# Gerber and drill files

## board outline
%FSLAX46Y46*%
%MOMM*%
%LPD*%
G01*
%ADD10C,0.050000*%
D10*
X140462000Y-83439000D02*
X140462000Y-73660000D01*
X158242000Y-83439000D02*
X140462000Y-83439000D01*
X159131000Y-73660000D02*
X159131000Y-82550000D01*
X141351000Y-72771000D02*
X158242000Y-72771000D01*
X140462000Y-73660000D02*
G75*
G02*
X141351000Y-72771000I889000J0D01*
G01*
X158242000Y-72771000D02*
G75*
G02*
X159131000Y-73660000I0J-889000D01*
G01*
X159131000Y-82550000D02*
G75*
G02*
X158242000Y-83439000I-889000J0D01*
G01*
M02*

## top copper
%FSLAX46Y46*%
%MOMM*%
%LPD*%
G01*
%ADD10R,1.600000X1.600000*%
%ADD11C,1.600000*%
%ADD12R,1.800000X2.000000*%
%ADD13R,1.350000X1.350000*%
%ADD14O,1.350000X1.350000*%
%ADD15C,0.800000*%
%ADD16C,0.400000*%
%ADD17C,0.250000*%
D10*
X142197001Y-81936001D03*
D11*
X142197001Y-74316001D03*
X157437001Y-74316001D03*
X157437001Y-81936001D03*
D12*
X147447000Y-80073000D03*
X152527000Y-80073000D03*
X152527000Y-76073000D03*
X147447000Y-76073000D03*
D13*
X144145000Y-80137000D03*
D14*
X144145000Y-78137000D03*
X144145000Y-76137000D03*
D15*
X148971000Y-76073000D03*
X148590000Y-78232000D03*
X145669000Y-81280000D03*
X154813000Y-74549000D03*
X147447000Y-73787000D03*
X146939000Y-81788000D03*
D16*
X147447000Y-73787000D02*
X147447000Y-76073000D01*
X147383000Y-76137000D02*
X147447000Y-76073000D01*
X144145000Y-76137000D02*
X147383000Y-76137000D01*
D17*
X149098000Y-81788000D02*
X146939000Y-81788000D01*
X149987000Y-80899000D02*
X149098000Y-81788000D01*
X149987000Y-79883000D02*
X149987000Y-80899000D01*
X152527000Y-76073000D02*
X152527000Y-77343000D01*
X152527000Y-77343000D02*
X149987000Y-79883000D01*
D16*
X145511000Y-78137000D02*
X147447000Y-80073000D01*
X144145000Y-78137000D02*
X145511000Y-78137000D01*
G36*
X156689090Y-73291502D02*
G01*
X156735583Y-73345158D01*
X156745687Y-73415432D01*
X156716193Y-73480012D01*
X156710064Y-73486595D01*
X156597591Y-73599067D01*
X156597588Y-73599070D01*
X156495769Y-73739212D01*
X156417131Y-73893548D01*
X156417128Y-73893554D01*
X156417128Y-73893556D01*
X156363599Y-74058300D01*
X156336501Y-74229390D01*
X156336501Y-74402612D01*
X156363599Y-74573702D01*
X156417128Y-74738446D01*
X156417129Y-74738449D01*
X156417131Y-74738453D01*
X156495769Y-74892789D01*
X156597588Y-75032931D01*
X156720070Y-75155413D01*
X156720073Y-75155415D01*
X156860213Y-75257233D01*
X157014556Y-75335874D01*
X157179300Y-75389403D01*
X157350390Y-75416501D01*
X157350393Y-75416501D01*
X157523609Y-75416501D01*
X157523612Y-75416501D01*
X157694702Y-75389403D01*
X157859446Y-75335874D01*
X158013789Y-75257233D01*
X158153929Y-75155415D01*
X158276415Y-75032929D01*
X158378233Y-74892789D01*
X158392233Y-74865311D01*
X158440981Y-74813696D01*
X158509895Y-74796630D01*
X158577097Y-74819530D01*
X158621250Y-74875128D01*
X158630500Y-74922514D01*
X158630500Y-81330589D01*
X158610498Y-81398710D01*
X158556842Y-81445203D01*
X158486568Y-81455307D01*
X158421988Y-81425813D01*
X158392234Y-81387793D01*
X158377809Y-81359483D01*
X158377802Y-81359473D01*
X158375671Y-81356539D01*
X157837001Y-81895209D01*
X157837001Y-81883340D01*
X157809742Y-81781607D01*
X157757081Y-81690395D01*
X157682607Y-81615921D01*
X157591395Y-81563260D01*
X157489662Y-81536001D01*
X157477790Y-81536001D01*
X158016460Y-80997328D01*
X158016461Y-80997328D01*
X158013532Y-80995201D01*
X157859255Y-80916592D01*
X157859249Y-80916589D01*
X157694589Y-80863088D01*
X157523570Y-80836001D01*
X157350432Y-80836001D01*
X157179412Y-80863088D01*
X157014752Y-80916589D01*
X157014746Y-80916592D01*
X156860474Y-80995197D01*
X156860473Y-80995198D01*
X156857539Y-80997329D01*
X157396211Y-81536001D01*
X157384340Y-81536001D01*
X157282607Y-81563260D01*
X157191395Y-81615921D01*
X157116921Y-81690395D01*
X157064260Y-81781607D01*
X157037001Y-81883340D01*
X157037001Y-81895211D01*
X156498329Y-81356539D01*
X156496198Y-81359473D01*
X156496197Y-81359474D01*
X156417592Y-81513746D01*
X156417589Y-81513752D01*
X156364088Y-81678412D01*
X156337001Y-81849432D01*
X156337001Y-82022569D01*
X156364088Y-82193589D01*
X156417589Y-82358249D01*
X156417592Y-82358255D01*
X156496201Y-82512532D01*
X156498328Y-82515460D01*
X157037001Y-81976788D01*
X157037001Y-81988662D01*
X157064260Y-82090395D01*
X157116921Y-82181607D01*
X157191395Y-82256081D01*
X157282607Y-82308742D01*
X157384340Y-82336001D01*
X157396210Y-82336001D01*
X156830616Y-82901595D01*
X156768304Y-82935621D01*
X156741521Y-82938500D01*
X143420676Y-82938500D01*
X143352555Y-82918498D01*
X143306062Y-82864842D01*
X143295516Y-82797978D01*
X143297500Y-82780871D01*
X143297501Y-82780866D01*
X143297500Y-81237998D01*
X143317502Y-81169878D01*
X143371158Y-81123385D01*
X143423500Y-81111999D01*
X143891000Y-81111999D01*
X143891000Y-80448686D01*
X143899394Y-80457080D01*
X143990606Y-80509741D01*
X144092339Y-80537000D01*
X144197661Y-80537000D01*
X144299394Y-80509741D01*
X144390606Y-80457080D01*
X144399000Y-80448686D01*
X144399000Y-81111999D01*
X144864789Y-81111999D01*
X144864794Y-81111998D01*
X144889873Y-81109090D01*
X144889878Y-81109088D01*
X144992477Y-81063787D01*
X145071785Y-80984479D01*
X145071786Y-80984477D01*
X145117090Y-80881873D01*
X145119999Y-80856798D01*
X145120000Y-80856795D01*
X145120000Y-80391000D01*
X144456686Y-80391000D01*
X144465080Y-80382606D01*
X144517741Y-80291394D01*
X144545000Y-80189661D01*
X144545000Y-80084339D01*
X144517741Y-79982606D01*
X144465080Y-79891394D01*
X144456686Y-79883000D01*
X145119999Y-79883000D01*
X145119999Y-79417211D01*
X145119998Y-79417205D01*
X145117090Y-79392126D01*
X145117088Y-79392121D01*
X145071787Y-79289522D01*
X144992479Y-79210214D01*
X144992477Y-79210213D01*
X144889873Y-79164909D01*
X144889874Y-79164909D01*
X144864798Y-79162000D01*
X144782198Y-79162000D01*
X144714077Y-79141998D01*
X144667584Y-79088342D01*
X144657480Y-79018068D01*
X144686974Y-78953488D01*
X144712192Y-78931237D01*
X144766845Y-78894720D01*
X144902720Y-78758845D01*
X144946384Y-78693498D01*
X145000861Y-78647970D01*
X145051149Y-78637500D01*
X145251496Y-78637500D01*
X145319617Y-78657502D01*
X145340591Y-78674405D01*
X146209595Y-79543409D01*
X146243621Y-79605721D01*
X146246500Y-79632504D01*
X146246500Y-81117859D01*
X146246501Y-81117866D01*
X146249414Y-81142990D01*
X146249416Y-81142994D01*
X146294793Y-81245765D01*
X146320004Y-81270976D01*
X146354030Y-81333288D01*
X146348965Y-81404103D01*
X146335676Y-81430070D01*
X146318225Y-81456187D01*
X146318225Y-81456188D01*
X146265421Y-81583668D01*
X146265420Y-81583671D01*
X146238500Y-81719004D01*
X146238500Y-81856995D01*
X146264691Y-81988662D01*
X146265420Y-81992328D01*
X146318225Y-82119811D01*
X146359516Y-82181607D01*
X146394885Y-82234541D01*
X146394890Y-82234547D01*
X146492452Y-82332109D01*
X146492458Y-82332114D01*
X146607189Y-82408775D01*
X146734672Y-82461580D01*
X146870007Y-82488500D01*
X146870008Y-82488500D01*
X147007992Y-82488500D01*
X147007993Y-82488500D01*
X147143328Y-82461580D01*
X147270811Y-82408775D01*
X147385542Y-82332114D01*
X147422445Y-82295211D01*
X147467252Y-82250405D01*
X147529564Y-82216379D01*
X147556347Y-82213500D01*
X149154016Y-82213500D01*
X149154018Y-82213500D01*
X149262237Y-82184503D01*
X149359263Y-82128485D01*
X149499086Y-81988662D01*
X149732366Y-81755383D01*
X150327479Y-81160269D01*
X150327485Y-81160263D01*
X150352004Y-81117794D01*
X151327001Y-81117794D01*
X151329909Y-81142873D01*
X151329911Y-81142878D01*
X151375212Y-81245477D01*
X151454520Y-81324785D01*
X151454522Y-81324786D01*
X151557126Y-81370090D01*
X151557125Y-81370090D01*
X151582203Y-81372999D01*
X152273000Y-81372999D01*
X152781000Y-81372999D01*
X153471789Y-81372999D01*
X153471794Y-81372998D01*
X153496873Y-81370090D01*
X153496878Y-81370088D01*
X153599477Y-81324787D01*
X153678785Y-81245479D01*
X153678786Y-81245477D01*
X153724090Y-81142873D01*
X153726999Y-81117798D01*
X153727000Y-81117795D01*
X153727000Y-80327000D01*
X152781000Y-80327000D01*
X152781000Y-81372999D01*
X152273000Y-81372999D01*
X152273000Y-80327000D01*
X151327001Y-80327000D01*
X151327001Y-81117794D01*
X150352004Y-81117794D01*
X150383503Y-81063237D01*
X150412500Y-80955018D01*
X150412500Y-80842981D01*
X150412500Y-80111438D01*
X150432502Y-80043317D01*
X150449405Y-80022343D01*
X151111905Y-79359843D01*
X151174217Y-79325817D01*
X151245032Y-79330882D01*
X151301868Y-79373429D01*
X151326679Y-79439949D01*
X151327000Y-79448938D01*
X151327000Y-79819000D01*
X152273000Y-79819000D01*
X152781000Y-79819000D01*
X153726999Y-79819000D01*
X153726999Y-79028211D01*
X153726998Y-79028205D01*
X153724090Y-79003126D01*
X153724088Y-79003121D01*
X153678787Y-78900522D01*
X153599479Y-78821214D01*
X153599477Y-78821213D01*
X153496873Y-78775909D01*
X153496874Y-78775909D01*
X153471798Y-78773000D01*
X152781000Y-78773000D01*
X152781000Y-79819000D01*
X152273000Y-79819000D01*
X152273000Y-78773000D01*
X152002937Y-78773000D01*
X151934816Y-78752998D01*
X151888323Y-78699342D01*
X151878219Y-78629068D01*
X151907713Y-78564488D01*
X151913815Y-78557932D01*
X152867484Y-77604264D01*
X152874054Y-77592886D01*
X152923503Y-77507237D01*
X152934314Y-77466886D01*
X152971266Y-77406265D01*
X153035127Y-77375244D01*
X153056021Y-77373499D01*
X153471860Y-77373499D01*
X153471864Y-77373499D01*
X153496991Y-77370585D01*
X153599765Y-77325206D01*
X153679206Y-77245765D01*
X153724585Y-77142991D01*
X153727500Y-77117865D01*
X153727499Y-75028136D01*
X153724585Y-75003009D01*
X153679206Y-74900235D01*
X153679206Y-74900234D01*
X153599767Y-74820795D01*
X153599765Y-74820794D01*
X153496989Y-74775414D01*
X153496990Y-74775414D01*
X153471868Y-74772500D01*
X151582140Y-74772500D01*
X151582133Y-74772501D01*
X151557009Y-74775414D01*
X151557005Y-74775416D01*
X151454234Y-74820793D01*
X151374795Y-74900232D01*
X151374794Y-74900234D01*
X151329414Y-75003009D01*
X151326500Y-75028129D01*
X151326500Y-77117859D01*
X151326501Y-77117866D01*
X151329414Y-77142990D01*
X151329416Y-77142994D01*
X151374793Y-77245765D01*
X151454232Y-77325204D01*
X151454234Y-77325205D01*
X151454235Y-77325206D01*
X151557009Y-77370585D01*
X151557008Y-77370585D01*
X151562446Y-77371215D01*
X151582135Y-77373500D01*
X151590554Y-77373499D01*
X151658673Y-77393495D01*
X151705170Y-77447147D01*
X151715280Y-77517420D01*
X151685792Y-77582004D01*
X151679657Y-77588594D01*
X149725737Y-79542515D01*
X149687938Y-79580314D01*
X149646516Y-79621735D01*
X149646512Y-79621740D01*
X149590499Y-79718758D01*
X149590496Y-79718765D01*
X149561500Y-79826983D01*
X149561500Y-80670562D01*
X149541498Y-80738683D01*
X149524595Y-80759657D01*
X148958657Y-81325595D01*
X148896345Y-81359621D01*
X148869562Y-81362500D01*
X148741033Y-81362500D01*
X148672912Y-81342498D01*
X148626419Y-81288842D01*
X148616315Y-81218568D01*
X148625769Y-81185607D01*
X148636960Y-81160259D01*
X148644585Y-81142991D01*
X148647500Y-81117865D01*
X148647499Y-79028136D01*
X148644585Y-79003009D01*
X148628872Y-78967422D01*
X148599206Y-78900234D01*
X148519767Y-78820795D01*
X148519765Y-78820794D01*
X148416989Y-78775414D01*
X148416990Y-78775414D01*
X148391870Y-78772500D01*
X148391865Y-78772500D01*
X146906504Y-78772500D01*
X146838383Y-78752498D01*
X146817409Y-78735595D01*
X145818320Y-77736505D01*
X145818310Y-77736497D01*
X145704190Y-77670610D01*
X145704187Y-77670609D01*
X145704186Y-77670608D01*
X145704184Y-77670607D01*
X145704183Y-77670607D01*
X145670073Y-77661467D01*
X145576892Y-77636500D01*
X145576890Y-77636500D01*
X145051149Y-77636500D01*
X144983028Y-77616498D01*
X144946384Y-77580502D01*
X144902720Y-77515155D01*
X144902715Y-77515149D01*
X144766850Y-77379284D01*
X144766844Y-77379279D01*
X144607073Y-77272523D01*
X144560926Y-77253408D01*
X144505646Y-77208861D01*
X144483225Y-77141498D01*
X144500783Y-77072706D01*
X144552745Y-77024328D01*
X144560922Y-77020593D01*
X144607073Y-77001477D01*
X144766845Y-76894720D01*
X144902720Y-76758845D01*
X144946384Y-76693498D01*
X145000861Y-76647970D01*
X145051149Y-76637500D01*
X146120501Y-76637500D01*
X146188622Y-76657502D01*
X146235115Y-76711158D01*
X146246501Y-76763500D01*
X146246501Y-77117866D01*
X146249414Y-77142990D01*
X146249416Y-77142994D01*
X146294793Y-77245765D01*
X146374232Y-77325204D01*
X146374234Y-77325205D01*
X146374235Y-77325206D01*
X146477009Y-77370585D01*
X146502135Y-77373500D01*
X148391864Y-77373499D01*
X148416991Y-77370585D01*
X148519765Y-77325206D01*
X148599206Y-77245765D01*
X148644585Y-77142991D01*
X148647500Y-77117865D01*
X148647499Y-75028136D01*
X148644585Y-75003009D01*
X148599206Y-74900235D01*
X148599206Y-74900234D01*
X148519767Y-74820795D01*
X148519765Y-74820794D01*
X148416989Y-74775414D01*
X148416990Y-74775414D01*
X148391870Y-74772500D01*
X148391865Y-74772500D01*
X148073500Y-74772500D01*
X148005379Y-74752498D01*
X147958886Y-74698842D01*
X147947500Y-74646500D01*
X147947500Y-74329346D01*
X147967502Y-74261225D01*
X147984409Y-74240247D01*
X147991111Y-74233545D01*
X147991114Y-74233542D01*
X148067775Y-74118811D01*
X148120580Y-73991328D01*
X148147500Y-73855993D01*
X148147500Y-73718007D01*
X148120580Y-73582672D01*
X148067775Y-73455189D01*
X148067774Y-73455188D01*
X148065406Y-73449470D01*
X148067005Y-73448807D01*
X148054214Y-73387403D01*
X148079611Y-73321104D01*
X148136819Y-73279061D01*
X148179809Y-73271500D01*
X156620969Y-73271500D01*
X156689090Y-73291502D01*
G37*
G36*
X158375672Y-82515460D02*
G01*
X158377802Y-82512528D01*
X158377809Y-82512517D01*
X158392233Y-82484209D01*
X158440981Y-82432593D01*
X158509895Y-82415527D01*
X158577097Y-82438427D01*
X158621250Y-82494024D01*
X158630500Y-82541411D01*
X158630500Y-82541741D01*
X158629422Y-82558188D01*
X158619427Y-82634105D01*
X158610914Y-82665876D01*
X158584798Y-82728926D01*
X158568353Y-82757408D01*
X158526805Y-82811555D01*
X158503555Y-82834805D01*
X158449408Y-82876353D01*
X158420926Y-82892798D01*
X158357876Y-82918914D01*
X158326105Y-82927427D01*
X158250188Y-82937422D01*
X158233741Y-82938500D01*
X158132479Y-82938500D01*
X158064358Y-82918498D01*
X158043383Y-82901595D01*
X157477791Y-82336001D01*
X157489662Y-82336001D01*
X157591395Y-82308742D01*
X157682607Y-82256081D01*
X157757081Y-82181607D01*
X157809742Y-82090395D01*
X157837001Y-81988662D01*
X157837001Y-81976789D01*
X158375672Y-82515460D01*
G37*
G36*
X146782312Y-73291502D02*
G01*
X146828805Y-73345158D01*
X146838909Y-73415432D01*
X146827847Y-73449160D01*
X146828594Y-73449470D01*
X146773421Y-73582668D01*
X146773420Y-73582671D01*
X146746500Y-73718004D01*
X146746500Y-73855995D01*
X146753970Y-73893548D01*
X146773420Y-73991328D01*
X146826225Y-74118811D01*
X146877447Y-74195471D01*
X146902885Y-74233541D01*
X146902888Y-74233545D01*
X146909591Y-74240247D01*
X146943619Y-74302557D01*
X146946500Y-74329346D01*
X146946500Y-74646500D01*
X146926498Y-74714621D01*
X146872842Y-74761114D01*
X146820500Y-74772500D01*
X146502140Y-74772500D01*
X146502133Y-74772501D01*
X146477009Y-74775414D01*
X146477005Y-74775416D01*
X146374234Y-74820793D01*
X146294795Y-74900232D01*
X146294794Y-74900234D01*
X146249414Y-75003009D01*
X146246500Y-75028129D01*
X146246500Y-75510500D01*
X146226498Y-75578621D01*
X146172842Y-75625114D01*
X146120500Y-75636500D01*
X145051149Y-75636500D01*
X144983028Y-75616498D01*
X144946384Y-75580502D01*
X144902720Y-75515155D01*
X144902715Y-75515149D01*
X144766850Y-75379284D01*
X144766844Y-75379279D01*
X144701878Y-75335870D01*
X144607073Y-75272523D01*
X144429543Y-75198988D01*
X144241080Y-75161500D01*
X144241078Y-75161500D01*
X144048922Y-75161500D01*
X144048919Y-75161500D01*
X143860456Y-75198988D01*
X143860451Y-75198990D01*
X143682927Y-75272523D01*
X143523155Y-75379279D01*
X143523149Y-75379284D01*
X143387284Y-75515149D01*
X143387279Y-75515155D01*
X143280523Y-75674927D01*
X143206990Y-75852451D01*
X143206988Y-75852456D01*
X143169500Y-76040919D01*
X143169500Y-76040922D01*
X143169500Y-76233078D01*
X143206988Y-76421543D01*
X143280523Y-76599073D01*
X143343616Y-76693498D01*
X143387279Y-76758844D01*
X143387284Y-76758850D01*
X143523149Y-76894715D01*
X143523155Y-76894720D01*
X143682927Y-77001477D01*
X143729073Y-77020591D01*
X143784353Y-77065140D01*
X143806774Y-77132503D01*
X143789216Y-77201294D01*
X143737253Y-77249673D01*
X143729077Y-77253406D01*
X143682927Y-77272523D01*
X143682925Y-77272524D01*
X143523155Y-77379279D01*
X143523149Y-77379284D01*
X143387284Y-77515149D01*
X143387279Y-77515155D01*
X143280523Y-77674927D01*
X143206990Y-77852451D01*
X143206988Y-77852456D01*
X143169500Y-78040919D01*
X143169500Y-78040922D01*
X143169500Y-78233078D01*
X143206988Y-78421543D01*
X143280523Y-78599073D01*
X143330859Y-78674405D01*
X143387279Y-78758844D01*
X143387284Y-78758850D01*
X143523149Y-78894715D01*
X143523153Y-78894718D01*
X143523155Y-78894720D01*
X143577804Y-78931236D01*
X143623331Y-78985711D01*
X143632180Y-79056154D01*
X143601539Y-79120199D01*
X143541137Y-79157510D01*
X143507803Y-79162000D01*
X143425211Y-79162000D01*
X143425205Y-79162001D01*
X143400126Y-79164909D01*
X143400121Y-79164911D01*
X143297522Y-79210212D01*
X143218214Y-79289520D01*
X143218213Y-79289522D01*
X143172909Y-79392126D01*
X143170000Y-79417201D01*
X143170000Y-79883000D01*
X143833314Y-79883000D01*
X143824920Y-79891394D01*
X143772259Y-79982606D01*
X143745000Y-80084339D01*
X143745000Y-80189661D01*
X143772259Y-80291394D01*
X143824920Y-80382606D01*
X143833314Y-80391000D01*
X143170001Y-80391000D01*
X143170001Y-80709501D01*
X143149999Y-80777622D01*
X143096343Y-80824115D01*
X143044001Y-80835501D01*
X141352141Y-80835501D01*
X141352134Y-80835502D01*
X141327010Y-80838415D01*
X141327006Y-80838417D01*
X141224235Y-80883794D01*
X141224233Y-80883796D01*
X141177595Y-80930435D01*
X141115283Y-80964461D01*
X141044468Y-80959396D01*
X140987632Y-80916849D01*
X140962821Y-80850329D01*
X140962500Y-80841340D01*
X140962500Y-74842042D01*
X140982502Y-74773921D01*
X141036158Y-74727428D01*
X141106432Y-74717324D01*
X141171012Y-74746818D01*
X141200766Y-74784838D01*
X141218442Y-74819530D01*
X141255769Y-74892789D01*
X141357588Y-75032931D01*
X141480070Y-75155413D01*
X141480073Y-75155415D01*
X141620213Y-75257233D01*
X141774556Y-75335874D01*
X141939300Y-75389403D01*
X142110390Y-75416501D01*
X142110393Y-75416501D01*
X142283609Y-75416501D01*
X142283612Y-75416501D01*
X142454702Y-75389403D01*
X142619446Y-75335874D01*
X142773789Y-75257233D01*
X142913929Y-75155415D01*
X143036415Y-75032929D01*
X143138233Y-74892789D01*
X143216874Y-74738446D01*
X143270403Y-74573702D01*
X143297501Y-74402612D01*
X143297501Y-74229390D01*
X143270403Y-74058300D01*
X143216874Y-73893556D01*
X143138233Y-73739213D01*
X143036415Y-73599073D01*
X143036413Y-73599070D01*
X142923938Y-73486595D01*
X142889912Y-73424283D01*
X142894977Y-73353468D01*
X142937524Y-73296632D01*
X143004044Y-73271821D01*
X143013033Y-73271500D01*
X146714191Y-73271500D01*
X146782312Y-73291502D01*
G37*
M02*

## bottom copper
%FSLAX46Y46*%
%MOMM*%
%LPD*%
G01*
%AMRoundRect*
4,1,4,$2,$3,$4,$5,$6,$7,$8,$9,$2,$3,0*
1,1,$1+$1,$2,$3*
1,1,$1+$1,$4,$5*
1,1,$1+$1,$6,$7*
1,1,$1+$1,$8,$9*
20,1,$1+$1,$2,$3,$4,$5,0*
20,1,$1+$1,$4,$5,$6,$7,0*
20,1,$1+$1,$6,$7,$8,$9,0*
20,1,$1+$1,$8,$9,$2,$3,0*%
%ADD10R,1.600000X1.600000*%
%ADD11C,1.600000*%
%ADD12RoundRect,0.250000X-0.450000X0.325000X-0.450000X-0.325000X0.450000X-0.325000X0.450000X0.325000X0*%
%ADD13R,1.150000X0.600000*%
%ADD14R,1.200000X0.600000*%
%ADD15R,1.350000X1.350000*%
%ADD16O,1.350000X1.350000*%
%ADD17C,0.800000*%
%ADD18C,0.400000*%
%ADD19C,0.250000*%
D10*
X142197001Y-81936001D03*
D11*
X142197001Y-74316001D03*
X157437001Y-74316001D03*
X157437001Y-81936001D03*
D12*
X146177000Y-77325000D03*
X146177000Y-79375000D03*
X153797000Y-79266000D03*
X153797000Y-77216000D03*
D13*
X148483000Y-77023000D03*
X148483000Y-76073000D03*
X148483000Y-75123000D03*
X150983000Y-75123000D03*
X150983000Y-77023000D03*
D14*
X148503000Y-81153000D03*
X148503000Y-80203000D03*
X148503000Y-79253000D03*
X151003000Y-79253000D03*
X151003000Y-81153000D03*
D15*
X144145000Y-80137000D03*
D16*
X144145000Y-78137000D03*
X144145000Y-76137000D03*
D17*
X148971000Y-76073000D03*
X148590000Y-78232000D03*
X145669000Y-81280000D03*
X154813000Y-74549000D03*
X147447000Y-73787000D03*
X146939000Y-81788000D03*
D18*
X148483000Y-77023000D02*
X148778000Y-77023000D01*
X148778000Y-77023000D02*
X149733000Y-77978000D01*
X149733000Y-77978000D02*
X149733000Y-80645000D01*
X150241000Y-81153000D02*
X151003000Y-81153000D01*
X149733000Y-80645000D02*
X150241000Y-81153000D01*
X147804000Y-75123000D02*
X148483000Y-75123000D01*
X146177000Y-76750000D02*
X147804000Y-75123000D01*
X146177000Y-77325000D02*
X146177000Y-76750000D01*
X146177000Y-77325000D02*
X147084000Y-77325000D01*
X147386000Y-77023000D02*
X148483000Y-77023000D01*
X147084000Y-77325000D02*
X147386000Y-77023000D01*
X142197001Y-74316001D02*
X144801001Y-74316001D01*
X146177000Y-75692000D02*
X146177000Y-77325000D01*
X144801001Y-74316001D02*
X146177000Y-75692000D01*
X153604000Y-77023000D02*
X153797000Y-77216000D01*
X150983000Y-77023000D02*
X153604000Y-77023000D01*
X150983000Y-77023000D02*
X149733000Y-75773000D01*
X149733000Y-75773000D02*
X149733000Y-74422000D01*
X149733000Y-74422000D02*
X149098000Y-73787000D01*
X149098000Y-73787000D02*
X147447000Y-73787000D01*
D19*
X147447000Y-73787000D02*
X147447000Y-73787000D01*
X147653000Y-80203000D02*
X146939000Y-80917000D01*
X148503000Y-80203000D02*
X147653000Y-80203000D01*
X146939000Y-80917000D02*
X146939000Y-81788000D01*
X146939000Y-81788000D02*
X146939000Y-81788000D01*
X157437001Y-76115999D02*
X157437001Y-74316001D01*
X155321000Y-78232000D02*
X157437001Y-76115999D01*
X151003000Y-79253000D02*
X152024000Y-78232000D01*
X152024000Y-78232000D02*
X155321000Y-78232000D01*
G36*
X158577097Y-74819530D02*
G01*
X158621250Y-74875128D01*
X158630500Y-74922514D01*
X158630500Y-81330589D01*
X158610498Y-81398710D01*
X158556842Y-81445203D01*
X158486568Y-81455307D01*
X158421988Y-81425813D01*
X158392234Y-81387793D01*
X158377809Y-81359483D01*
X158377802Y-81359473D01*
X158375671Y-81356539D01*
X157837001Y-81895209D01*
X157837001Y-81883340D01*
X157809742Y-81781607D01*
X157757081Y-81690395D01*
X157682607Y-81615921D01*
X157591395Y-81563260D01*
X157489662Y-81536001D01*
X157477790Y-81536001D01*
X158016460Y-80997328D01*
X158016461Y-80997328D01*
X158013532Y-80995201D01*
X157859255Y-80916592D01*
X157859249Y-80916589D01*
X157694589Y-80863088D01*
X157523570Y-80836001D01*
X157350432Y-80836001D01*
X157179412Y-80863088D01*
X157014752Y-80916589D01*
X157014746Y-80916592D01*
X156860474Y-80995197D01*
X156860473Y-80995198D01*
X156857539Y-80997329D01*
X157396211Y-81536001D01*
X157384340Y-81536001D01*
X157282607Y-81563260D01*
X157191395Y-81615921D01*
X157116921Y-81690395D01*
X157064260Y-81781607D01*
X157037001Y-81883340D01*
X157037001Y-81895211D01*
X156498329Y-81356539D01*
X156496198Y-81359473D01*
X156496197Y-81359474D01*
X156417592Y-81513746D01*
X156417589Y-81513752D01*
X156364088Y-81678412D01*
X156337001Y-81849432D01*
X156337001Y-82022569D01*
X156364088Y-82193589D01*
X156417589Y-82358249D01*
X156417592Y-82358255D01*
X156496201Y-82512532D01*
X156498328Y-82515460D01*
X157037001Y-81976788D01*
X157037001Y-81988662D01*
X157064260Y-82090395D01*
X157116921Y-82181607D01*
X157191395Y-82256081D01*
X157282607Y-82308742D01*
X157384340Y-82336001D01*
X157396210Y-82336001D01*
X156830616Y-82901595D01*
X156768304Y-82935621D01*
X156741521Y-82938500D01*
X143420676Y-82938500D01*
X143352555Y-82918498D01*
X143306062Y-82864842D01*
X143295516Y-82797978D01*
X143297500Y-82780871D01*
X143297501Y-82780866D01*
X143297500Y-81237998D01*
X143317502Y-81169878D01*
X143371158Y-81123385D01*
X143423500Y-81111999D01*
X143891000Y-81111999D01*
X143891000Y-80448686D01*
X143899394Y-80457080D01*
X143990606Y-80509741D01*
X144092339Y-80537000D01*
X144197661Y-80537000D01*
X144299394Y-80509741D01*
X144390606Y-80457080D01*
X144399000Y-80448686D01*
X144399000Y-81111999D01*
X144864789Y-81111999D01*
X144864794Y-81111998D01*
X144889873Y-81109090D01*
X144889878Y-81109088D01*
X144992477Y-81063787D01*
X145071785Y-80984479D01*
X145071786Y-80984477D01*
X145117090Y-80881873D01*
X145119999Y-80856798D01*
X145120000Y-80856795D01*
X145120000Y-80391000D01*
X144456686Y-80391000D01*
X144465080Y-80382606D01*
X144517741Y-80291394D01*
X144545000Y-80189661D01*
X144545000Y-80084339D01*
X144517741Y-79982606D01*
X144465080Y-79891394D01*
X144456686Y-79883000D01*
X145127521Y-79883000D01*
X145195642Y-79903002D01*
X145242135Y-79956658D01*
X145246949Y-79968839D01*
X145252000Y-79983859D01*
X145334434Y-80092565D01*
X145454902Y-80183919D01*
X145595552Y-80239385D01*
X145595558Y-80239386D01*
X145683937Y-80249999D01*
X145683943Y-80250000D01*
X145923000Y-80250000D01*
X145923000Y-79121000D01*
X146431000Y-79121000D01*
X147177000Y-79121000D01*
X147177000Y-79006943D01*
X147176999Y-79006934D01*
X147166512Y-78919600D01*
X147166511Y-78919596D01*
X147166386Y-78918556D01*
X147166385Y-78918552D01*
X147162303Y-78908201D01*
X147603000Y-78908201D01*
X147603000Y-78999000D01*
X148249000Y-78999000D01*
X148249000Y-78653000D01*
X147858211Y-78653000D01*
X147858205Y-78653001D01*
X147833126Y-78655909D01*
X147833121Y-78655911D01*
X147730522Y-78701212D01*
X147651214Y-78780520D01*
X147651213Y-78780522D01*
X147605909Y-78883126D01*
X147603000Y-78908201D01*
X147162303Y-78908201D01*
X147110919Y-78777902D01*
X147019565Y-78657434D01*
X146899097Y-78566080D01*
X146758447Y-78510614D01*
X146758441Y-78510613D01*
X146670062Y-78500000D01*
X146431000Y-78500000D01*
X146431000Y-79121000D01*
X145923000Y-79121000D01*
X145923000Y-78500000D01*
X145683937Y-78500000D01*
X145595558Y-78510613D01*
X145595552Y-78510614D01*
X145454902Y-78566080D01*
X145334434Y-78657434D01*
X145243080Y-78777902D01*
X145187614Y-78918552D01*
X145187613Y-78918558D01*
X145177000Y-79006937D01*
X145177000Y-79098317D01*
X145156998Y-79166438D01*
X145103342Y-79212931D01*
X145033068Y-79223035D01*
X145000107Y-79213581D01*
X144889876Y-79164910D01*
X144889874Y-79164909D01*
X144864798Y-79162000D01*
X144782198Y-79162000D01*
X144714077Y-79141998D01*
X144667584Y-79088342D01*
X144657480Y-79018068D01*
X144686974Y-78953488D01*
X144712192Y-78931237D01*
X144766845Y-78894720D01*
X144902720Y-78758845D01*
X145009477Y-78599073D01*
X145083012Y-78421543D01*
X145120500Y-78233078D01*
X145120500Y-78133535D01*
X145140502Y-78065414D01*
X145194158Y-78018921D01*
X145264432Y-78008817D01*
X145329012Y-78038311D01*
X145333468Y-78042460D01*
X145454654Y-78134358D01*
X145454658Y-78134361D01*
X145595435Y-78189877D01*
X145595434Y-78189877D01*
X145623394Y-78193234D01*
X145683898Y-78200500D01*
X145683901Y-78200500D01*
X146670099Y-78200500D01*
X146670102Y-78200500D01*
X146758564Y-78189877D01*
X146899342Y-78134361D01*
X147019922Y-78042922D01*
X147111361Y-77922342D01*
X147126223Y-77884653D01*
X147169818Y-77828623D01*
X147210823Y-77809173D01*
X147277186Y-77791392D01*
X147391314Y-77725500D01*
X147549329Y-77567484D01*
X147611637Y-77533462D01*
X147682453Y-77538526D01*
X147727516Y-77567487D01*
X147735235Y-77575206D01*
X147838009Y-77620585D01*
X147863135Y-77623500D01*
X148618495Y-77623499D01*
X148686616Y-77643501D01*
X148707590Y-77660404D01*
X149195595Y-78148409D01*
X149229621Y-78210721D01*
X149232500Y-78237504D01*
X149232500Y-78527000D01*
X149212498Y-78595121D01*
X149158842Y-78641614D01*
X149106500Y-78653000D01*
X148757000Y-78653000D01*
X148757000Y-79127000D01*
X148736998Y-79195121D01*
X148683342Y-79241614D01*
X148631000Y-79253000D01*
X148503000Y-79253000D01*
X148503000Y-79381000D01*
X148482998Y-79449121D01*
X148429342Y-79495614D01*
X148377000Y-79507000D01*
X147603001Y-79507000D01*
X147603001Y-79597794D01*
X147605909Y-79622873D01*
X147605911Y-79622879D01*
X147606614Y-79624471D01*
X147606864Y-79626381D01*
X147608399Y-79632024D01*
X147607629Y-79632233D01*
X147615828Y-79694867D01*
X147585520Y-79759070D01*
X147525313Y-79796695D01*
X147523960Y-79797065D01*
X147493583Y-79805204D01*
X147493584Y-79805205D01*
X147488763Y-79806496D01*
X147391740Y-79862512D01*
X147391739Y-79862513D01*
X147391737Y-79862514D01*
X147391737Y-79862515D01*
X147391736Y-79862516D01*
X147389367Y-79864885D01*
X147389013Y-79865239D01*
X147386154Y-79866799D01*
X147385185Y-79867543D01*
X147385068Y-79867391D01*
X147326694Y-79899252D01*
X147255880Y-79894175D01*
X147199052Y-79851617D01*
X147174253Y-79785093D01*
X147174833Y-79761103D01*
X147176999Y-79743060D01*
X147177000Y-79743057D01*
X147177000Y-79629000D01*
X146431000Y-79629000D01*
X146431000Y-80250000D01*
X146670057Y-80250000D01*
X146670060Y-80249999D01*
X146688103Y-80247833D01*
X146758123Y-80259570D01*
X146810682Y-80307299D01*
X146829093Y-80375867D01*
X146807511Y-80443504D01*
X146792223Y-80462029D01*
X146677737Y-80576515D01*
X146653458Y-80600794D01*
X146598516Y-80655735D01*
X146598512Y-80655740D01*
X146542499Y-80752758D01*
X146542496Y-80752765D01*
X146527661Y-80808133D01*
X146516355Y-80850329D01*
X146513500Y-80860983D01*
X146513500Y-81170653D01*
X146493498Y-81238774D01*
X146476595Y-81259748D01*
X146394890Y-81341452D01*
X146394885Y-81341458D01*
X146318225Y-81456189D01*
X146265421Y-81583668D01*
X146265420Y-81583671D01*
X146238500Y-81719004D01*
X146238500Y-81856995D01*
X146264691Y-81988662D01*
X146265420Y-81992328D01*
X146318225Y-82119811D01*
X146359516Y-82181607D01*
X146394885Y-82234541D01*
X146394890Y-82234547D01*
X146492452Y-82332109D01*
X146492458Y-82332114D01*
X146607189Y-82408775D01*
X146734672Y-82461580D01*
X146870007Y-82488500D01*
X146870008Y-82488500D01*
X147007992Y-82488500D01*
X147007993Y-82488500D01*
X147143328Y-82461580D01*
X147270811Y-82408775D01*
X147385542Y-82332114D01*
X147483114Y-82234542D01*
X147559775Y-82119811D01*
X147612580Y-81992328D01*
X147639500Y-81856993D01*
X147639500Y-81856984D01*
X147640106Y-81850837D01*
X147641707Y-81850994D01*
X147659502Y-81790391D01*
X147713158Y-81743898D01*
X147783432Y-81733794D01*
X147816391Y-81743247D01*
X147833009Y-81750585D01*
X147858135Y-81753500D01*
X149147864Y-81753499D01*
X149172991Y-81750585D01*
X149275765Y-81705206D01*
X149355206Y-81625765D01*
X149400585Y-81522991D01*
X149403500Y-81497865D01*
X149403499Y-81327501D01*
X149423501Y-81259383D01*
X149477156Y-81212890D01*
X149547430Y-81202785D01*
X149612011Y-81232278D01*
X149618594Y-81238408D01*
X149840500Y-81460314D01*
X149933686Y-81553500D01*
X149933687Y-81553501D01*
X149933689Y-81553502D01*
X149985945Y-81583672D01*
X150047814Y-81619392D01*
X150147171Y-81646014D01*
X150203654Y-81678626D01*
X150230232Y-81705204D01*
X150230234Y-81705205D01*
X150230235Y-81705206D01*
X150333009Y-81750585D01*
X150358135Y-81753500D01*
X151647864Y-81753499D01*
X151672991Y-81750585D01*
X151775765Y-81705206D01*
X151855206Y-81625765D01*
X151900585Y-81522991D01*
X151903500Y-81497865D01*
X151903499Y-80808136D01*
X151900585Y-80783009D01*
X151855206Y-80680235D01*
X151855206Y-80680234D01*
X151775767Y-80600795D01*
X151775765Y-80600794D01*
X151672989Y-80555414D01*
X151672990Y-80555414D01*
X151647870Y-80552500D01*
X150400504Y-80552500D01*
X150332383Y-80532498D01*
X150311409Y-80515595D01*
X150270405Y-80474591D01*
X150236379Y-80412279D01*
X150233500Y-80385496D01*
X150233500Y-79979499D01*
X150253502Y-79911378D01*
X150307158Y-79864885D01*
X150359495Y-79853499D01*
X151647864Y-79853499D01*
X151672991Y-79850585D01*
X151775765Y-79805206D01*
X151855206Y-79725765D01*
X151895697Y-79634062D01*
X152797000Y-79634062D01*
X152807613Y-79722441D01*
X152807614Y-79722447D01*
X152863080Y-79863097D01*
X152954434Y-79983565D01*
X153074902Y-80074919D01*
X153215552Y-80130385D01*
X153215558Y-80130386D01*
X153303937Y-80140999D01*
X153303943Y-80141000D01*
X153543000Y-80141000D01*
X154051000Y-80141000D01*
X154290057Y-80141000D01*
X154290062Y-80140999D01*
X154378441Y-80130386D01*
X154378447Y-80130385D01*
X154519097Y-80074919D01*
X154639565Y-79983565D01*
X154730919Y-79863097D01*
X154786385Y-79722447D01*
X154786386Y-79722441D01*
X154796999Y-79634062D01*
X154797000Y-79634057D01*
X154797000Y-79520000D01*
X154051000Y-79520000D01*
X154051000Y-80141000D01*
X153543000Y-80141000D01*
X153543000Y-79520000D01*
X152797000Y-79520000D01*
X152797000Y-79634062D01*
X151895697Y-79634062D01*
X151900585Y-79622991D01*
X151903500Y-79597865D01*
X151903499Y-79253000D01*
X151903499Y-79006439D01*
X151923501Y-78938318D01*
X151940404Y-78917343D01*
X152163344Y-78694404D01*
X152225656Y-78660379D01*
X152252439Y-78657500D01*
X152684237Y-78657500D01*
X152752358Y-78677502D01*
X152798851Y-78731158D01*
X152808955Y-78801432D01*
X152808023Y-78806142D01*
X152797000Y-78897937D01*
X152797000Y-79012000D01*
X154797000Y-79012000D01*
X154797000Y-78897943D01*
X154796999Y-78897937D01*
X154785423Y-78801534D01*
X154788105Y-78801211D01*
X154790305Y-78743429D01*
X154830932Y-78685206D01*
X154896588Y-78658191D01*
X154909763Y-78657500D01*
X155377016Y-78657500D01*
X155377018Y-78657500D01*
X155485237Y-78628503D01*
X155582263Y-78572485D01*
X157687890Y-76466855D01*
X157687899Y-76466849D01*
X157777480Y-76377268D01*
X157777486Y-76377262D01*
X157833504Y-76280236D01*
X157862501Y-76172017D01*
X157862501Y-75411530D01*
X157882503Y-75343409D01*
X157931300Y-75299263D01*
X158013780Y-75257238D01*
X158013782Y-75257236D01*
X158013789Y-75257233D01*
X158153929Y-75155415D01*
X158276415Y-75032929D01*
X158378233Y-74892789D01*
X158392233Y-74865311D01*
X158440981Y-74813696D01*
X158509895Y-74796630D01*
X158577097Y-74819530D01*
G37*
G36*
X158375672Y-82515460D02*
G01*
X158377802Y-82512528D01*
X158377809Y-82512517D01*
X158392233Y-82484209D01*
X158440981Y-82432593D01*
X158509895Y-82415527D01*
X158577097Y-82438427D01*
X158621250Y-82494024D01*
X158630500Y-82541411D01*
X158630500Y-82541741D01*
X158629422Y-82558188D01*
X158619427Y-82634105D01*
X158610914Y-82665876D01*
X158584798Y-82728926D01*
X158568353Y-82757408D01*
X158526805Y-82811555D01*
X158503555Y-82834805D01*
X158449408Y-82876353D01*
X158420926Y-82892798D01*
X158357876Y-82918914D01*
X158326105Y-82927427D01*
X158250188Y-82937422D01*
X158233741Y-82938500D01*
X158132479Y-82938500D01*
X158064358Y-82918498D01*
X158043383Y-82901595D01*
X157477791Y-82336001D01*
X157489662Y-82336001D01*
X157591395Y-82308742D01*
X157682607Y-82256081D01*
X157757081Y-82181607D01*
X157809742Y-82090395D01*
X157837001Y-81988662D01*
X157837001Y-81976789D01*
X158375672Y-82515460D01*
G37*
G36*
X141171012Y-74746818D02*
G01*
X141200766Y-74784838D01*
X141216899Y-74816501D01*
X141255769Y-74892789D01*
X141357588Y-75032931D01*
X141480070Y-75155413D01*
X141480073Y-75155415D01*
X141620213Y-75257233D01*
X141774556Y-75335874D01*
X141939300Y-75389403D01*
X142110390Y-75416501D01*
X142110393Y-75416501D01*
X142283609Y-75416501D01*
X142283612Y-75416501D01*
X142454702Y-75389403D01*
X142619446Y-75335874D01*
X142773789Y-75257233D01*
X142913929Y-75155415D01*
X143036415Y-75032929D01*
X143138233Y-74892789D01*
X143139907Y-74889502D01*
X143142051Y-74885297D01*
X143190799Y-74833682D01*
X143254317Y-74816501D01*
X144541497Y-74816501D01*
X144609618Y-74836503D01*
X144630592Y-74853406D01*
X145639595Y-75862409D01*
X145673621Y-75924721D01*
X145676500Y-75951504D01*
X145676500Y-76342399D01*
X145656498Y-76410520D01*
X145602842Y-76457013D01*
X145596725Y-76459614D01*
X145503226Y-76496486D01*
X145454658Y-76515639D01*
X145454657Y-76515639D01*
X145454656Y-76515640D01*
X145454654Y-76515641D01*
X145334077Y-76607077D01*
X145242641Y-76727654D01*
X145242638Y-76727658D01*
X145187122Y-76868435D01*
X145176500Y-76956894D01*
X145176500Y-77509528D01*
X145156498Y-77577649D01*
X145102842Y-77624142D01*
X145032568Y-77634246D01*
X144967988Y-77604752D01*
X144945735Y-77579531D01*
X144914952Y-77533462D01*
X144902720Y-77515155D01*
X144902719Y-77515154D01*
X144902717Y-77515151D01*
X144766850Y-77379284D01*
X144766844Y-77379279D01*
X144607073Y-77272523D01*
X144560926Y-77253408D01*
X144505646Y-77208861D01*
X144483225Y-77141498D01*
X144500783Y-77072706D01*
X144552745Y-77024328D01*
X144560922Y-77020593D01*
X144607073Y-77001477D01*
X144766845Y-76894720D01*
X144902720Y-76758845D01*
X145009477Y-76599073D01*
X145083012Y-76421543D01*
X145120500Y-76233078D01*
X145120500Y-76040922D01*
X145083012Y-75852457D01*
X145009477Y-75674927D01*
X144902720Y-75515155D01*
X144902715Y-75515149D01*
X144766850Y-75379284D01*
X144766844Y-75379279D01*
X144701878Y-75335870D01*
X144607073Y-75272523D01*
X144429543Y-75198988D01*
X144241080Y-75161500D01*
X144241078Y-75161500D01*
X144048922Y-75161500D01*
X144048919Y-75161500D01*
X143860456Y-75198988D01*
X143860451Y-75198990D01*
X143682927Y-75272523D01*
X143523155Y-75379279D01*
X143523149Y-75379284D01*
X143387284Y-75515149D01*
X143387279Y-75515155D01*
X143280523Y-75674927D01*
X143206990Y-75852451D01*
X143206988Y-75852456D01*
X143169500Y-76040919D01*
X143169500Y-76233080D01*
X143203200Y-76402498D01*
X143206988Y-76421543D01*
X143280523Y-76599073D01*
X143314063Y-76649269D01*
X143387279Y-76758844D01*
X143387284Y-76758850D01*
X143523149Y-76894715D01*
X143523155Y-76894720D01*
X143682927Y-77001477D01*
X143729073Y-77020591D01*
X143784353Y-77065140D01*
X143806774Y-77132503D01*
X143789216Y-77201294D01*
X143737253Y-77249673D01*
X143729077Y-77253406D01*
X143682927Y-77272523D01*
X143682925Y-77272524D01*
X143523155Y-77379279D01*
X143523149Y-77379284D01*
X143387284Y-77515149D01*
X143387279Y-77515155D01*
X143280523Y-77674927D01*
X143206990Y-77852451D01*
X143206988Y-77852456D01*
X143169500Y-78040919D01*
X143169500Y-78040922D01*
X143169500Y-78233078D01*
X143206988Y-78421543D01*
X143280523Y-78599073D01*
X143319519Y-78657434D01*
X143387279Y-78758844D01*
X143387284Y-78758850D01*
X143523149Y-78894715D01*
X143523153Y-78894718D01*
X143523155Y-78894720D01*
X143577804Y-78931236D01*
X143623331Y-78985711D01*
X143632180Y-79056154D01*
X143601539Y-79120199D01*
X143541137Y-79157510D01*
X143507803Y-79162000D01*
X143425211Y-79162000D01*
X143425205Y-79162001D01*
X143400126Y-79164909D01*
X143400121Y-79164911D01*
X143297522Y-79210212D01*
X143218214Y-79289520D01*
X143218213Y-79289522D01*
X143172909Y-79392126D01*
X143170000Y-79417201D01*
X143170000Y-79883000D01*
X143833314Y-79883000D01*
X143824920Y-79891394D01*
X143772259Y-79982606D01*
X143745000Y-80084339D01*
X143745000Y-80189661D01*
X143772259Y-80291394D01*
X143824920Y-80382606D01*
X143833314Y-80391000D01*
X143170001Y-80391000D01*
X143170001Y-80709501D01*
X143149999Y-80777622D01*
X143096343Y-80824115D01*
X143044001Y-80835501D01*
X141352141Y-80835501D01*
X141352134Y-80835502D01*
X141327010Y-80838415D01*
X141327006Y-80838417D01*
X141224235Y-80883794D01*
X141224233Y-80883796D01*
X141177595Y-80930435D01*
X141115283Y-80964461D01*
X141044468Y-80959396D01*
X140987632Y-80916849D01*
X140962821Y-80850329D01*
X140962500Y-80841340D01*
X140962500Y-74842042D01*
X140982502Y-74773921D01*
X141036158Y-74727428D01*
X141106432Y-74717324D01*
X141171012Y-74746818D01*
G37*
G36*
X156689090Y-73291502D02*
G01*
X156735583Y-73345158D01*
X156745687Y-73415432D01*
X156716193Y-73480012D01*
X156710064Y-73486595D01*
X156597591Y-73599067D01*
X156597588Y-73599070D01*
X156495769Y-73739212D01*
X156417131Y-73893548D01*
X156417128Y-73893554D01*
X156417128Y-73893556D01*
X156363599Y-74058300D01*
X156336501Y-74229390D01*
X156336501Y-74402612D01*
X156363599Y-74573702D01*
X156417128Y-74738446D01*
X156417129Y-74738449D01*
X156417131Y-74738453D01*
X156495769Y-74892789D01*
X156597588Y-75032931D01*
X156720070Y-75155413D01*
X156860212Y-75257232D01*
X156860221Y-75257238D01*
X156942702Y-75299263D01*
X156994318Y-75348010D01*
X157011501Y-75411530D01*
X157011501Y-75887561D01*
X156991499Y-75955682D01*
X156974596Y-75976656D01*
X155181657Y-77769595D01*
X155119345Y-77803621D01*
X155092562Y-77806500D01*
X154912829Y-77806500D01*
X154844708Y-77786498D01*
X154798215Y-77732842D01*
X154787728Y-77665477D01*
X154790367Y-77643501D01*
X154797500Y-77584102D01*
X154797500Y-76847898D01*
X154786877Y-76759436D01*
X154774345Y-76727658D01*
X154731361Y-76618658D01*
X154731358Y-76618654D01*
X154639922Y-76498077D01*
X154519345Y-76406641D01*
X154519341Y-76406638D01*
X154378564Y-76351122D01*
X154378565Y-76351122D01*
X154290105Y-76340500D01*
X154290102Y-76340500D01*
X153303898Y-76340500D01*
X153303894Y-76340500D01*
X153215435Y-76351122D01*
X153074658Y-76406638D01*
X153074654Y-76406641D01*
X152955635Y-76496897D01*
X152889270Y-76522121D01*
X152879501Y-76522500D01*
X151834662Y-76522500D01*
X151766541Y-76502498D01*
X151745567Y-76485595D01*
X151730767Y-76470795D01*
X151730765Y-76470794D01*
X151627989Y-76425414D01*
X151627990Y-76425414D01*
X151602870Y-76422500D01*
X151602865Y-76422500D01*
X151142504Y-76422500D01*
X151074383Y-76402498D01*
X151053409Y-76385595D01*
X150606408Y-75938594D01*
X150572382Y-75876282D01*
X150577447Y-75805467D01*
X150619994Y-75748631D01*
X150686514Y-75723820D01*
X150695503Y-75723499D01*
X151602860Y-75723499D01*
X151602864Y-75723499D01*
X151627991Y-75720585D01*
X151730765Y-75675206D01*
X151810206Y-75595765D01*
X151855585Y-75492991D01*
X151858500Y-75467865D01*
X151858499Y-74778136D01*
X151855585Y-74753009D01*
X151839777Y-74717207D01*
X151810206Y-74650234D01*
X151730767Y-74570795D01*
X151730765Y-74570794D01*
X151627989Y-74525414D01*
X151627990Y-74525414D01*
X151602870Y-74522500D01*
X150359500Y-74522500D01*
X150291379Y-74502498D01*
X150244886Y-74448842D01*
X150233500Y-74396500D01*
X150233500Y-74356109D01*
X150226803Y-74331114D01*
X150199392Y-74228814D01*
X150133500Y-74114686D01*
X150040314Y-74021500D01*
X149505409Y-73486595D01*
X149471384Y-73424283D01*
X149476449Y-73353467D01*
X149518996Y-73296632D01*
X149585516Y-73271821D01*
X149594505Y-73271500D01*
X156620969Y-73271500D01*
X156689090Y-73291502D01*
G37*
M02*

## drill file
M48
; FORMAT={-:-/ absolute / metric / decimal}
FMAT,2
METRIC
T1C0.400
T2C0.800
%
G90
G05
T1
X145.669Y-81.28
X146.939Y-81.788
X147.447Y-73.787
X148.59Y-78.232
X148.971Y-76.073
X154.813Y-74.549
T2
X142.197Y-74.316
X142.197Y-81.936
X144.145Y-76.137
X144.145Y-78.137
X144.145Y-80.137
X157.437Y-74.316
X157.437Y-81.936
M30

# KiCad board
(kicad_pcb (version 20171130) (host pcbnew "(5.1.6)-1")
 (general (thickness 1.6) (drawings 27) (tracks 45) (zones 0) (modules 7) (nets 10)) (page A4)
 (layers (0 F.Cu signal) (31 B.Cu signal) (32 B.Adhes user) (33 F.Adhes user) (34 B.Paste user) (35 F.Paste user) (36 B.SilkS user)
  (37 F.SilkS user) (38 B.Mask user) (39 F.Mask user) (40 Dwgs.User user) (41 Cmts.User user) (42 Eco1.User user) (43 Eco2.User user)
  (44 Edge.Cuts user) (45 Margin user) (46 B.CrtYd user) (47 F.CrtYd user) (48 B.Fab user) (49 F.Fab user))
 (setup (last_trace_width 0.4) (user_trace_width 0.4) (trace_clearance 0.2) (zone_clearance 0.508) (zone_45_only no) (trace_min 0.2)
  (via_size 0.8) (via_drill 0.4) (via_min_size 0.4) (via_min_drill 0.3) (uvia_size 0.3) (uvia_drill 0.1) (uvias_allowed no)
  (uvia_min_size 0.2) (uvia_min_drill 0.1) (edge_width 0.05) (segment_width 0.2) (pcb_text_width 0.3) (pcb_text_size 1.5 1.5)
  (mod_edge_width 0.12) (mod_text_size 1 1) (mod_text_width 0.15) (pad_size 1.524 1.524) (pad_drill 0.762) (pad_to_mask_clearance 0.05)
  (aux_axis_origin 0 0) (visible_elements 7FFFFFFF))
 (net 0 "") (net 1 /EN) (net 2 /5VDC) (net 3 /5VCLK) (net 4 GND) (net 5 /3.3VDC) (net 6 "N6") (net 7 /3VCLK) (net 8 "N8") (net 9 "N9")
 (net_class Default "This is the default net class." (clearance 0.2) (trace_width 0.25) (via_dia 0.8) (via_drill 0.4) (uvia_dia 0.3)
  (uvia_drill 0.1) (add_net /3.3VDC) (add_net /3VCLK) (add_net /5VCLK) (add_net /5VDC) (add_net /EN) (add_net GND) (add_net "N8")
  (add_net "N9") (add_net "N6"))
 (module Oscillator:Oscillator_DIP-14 (layer F.Cu) (at 142.197001 81.936001)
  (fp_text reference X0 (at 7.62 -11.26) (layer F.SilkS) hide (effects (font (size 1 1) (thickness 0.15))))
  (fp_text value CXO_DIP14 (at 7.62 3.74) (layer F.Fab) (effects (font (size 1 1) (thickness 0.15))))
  (pad 1 thru_hole rect (at 0 0) (size 1.6 1.6) (drill 0.8) (layers *.Cu *.Mask) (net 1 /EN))
  (pad 14 thru_hole circle (at 0 -7.62) (size 1.6 1.6) (drill 0.8) (layers *.Cu *.Mask) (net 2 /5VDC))
  (pad 8 thru_hole circle (at 15.24 -7.62) (size 1.6 1.6) (drill 0.8) (layers *.Cu *.Mask) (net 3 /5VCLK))
  (pad 7 thru_hole circle (at 15.24 0) (size 1.6 1.6) (drill 0.8) (layers *.Cu *.Mask) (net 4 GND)))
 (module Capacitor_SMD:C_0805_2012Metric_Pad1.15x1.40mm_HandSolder (layer B.Cu) (at 146.177 78.35 270)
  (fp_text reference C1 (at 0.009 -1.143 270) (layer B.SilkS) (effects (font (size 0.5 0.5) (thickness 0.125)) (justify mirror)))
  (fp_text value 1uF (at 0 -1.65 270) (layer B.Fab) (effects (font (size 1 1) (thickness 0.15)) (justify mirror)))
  (pad 1 smd roundrect (at -1.025 0 270) (size 1.15 1.4) (layers B.Cu B.Paste B.Mask) (roundrect_rratio 0.217391) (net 2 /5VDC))
  (pad 2 smd roundrect (at 1.025 0 270) (size 1.15 1.4) (layers B.Cu B.Paste B.Mask) (roundrect_rratio 0.217391) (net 4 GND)))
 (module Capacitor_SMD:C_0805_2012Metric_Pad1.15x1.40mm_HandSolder (layer B.Cu) (at 153.797 78.241 270)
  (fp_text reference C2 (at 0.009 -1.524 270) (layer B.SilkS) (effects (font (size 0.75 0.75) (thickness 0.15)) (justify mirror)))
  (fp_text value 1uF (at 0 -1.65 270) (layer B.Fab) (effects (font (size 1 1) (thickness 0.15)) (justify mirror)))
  (pad 2 smd roundrect (at 1.025 0 270) (size 1.15 1.4) (layers B.Cu B.Paste B.Mask) (roundrect_rratio 0.217391) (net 4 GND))
  (pad 1 smd roundrect (at -1.025 0 270) (size 1.15 1.4) (layers B.Cu B.Paste B.Mask) (roundrect_rratio 0.217391) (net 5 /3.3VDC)))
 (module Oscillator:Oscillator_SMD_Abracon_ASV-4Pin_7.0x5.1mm (layer F.Cu) (at 149.987 78.073)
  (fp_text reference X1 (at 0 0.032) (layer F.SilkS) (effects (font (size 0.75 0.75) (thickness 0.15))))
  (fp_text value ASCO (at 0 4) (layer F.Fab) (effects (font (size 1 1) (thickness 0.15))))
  (pad 1 smd rect (at -2.54 2) (size 1.8 2) (layers F.Cu F.Paste F.Mask) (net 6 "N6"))
  (pad 2 smd rect (at 2.54 2) (size 1.8 2) (layers F.Cu F.Paste F.Mask) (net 4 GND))
  (pad 3 smd rect (at 2.54 -2) (size 1.8 2) (layers F.Cu F.Paste F.Mask) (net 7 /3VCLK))
  (pad 4 smd rect (at -2.54 -2) (size 1.8 2) (layers F.Cu F.Paste F.Mask) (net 5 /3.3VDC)))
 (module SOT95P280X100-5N (layer B.Cu) (at 149.733 76.073)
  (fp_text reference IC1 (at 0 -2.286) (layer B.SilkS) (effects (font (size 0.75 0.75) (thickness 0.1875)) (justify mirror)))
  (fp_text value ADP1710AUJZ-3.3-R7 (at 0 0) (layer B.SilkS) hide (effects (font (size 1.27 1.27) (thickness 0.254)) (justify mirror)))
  (pad 1 smd rect (at -1.25 0.95 270) (size 0.6 1.15) (layers B.Cu B.Paste B.Mask) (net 2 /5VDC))
  (pad 2 smd rect (at -1.25 0 270) (size 0.6 1.15) (layers B.Cu B.Paste B.Mask) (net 4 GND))
  (pad 3 smd rect (at -1.25 -0.95 270) (size 0.6 1.15) (layers B.Cu B.Paste B.Mask) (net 2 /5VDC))
  (pad 4 smd rect (at 1.25 -0.95 270) (size 0.6 1.15) (layers B.Cu B.Paste B.Mask) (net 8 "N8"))
  (pad 5 smd rect (at 1.25 0.95 270) (size 0.6 1.15) (layers B.Cu B.Paste B.Mask) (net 5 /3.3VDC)))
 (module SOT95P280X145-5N (layer B.Cu) (at 149.753 80.203)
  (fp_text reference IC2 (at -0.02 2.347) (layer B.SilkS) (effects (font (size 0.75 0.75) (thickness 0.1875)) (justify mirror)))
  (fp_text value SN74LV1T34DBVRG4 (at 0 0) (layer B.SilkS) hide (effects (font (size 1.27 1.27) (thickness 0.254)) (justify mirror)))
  (pad 1 smd rect (at -1.25 0.95 270) (size 0.6 1.2) (layers B.Cu B.Paste B.Mask) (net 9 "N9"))
  (pad 2 smd rect (at -1.25 0 270) (size 0.6 1.2) (layers B.Cu B.Paste B.Mask) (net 7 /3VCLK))
  (pad 3 smd rect (at -1.25 -0.95 270) (size 0.6 1.2) (layers B.Cu B.Paste B.Mask) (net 4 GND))
  (pad 4 smd rect (at 1.25 -0.95 270) (size 0.6 1.2) (layers B.Cu B.Paste B.Mask) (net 3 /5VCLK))
  (pad 5 smd rect (at 1.25 0.95 270) (size 0.6 1.2) (layers B.Cu B.Paste B.Mask) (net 2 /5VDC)))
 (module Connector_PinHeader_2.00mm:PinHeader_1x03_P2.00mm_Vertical (layer F.Cu) (at 144.145 80.137 180)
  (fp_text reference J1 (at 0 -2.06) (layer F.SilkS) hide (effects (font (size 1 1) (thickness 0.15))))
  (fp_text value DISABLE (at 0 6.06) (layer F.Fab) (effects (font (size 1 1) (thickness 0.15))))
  (pad 1 thru_hole rect (at 0 0 180) (size 1.35 1.35) (drill 0.8) (layers *.Cu *.Mask) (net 4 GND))
  (pad 2 thru_hole oval (at 0 2 180) (size 1.35 1.35) (drill 0.8) (layers *.Cu *.Mask) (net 6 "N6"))
  (pad 3 thru_hole oval (at 0 4 180) (size 1.35 1.35) (drill 0.8) (layers *.Cu *.Mask) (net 5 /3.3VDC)))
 (gr_line (start 140.462 83.439) (end 140.462 73.66) (layer Edge.Cuts) (width 0.05))
 (gr_line (start 158.242 83.439) (end 140.462 83.439) (layer Edge.Cuts) (width 0.05))
 (gr_line (start 159.131 73.66) (end 159.131 82.55) (layer Edge.Cuts) (width 0.05))
 (gr_line (start 141.351 72.771) (end 158.242 72.771) (layer Edge.Cuts) (width 0.05))
 (gr_arc (start 141.351 73.66) (end 141.351 72.771) (angle -90) (layer Edge.Cuts) (width 0.05))
 (gr_arc (start 158.242 73.66) (end 159.131 73.66) (angle -90) (layer Edge.Cuts) (width 0.05))
 (gr_arc (start 158.242 82.55) (end 158.242 83.439) (angle -90) (layer Edge.Cuts) (width 0.05))
 (segment (start 148.483 77.023) (end 148.778 77.023) (width 0.4) (layer B.Cu) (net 2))
 (segment (start 148.778 77.023) (end 149.733 77.978) (width 0.4) (layer B.Cu) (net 2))
 (segment (start 149.733 77.978) (end 149.733 80.645) (width 0.4) (layer B.Cu) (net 2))
 (segment (start 150.241 81.153) (end 151.003 81.153) (width 0.4) (layer B.Cu) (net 2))
 (segment (start 149.733 80.645) (end 150.241 81.153) (width 0.4) (layer B.Cu) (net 2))
 (segment (start 147.804 75.123) (end 148.483 75.123) (width 0.4) (layer B.Cu) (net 2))
 (segment (start 146.177 76.75) (end 147.804 75.123) (width 0.4) (layer B.Cu) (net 2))
 (segment (start 146.177 77.325) (end 146.177 76.75) (width 0.4) (layer B.Cu) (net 2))
 (segment (start 146.177 77.325) (end 147.084 77.325) (width 0.4) (layer B.Cu) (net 2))
 (segment (start 147.386 77.023) (end 148.483 77.023) (width 0.4) (layer B.Cu) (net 2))
 (segment (start 147.084 77.325) (end 147.386 77.023) (width 0.4) (layer B.Cu) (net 2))
 (segment (start 142.197001 74.316001) (end 144.801001 74.316001) (width 0.4) (layer B.Cu) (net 2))
 (segment (start 146.177 75.692) (end 146.177 77.325) (width 0.4) (layer B.Cu) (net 2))
 (segment (start 144.801001 74.316001) (end 146.177 75.692) (width 0.4) (layer B.Cu) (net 2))
 (via (at 148.971 76.073) (size 0.8) (drill 0.4) (layers F.Cu B.Cu) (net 4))
 (via (at 148.59 78.232) (size 0.8) (drill 0.4) (layers F.Cu B.Cu) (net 4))
 (via (at 145.669 81.28) (size 0.8) (drill 0.4) (layers F.Cu B.Cu) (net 4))
 (via (at 154.813 74.549) (size 0.8) (drill 0.4) (layers F.Cu B.Cu) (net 4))
 (segment (start 153.604 77.023) (end 153.797 77.216) (width 0.4) (layer B.Cu) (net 5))
 (segment (start 150.983 77.023) (end 153.604 77.023) (width 0.4) (layer B.Cu) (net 5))
 (segment (start 150.983 77.023) (end 149.733 75.773) (width 0.4) (layer B.Cu) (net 5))
 (segment (start 149.733 75.773) (end 149.733 74.422) (width 0.4) (layer B.Cu) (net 5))
 (segment (start 149.733 74.422) (end 149.098 73.787) (width 0.4) (layer B.Cu) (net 5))
 (segment (start 149.098 73.787) (end 147.447 73.787) (width 0.4) (layer B.Cu) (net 5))
 (segment (start 147.447 73.787) (end 147.447 73.787) (width 0.25) (layer B.Cu) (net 5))
 (via (at 147.447 73.787) (size 0.8) (drill 0.4) (layers F.Cu B.Cu) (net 5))
 (segment (start 147.447 73.787) (end 147.447 76.073) (width 0.4) (layer F.Cu) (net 5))
 (segment (start 147.383 76.137) (end 147.447 76.073) (width 0.4) (layer F.Cu) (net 5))
 (segment (start 144.145 76.137) (end 147.383 76.137) (width 0.4) (layer F.Cu) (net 5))
 (segment (start 147.653 80.203) (end 146.939 80.917) (width 0.25) (layer B.Cu) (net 7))
 (segment (start 148.503 80.203) (end 147.653 80.203) (width 0.25) (layer B.Cu) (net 7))
 (segment (start 146.939 80.917) (end 146.939 81.788) (width 0.25) (layer B.Cu) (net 7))
 (segment (start 146.939 81.788) (end 146.939 81.788) (width 0.25) (layer B.Cu) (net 7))
 (via (at 146.939 81.788) (size 0.8) (drill 0.4) (layers F.Cu B.Cu) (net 7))
 (segment (start 149.098 81.788) (end 146.939 81.788) (width 0.25) (layer F.Cu) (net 7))
 (segment (start 149.987 80.899) (end 149.098 81.788) (width 0.25) (layer F.Cu) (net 7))
 (segment (start 149.987 79.883) (end 149.987 80.899) (width 0.25) (layer F.Cu) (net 7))
 (segment (start 152.527 76.073) (end 152.527 77.343) (width 0.25) (layer F.Cu) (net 7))
 (segment (start 152.527 77.343) (end 149.987 79.883) (width 0.25) (layer F.Cu) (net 7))
 (segment (start 157.437001 76.115999) (end 157.437001 74.316001) (width 0.25) (layer B.Cu) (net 3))
 (segment (start 155.321 78.232) (end 157.437001 76.115999) (width 0.25) (layer B.Cu) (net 3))
 (segment (start 151.003 79.253) (end 152.024 78.232) (width 0.25) (layer B.Cu) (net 3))
 (segment (start 152.024 78.232) (end 155.321 78.232) (width 0.25) (layer B.Cu) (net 3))
 (segment (start 145.511 78.137) (end 147.447 80.073) (width 0.4) (layer F.Cu) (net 6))
 (segment (start 144.145 78.137) (end 145.511 78.137) (width 0.4) (layer F.Cu) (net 6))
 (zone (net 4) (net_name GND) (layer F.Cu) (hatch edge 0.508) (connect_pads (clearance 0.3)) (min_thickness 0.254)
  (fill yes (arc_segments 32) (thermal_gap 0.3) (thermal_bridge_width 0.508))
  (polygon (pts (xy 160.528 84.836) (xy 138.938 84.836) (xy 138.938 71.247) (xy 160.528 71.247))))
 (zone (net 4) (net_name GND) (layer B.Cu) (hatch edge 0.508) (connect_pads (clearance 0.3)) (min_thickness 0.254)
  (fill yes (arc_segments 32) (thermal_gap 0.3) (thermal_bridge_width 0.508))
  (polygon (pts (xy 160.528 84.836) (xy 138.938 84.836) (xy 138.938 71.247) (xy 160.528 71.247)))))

